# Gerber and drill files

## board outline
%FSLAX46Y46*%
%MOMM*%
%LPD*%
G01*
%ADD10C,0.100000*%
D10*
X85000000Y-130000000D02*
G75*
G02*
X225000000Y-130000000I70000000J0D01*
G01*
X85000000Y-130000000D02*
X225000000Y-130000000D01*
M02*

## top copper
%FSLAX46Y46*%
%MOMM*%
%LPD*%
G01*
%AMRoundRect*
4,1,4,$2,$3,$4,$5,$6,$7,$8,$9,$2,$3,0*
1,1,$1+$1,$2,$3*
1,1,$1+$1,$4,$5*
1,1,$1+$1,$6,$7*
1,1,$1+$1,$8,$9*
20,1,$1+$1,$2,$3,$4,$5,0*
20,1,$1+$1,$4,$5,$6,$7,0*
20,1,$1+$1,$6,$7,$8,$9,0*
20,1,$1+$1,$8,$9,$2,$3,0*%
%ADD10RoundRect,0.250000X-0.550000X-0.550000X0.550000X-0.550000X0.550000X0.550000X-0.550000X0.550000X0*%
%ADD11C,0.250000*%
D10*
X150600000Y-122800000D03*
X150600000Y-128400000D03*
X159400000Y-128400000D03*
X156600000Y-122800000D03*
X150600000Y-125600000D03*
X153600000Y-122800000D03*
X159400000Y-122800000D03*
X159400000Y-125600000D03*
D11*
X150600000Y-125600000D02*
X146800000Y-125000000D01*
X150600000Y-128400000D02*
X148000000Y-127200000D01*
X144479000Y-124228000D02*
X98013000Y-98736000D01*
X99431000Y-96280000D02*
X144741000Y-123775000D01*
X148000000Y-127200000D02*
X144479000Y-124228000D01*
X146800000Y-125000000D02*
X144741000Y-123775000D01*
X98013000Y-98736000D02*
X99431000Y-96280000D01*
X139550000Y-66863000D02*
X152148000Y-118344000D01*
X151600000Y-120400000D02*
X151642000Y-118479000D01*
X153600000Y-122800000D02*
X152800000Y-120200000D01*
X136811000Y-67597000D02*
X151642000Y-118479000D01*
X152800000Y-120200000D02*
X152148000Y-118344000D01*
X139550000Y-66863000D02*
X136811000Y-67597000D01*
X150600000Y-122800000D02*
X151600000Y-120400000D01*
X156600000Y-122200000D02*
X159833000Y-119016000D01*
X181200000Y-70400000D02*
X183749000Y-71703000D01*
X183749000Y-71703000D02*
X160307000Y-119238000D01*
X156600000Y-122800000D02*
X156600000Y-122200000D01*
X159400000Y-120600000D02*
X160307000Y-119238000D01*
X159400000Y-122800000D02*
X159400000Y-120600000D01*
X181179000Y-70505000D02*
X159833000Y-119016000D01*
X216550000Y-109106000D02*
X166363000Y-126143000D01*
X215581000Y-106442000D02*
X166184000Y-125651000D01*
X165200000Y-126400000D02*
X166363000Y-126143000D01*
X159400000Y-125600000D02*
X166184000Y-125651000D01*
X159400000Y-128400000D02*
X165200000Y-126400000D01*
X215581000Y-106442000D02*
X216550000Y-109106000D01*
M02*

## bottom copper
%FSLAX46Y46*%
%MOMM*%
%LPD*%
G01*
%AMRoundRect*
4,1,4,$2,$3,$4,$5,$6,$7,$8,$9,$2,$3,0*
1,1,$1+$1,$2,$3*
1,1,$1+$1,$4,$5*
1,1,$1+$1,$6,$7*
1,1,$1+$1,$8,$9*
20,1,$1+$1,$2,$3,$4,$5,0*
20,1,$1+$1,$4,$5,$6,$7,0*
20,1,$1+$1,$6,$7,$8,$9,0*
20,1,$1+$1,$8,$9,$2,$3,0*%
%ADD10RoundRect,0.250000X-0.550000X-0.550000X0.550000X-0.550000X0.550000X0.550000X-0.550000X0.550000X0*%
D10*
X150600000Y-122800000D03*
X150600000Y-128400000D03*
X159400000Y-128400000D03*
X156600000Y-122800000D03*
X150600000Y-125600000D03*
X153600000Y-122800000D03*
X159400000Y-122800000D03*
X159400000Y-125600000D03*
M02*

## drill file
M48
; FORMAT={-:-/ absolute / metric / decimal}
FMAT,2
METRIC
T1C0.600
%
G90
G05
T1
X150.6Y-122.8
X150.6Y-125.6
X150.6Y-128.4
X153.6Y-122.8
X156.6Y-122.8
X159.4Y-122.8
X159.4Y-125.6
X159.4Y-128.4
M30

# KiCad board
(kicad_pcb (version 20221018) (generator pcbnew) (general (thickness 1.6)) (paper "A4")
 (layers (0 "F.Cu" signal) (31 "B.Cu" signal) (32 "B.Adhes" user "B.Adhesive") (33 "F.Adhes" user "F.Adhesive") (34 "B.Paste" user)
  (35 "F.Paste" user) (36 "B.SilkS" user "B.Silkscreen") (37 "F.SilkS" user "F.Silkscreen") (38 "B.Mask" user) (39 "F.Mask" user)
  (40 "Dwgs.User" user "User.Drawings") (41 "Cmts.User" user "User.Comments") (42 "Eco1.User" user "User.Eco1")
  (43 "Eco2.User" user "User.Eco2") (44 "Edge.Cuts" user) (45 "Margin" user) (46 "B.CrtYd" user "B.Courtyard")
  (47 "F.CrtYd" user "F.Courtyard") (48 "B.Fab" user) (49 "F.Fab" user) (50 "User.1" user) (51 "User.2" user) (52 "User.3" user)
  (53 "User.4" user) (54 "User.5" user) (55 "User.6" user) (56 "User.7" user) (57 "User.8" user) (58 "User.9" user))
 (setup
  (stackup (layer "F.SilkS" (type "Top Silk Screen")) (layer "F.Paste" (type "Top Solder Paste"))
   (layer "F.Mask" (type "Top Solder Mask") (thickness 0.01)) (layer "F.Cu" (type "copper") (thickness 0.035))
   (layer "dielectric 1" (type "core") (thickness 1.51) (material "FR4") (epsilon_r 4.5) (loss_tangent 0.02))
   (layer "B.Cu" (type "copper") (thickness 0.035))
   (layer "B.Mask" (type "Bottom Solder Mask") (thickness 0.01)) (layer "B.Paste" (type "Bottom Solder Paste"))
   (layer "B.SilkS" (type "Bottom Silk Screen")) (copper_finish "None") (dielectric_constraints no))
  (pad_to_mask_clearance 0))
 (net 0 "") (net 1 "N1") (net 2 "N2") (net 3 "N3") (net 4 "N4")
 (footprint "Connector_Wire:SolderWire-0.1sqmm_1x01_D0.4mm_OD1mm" (layer "F.Cu") (at 150.6 122.8)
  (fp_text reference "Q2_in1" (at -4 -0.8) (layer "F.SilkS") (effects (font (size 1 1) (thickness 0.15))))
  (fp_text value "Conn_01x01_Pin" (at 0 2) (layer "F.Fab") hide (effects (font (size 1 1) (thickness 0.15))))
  (pad "1" thru_hole roundrect (at 0 0) (size 1.6 1.6) (drill 0.6) (layers "*.Cu" "*.Mask") (roundrect_rratio 0.15625) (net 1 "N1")))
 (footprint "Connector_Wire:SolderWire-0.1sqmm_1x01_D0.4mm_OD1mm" (layer "F.Cu") (at 150.6 128.4)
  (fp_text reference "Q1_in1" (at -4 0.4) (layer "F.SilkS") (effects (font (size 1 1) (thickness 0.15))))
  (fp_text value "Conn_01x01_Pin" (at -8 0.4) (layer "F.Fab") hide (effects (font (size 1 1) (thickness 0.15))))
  (pad "1" thru_hole roundrect (at 0 0) (size 1.6 1.6) (drill 0.6) (layers "*.Cu" "*.Mask") (roundrect_rratio 0.15625) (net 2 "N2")))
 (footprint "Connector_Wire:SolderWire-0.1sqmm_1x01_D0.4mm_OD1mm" (layer "F.Cu") (at 159.4 128.4)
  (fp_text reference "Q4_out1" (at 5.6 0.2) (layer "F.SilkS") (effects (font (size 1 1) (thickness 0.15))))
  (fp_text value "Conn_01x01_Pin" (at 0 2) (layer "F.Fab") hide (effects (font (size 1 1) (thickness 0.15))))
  (pad "1" thru_hole roundrect (at 0 0) (size 1.6 1.6) (drill 0.6) (layers "*.Cu" "*.Mask") (roundrect_rratio 0.15625) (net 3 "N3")))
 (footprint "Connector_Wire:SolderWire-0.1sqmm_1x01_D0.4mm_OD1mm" (layer "F.Cu") (at 156.6 122.8)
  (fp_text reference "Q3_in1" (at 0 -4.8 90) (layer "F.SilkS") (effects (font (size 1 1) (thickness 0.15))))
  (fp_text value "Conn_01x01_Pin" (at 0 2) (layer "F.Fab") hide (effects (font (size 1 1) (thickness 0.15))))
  (pad "1" thru_hole roundrect (at 0 0) (size 1.6 1.6) (drill 0.6) (layers "*.Cu" "*.Mask") (roundrect_rratio 0.15625) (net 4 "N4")))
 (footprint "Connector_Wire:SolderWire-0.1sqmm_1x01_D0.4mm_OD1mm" (layer "F.Cu") (at 150.6 125.6)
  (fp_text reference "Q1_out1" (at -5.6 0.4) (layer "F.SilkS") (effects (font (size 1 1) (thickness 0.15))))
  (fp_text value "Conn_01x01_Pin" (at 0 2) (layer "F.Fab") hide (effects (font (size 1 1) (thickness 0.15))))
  (pad "1" thru_hole roundrect (at 0 0) (size 1.6 1.6) (drill 0.6) (layers "*.Cu" "*.Mask") (roundrect_rratio 0.15625) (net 2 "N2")))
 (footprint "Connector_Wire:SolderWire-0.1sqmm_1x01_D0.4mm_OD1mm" (layer "F.Cu") (at 153.6 122.8)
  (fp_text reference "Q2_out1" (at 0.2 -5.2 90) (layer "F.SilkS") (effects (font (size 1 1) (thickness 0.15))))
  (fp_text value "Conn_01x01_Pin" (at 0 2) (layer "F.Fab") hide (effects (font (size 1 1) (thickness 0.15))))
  (pad "1" thru_hole roundrect (at 0 0) (size 1.6 1.6) (drill 0.6) (layers "*.Cu" "*.Mask") (roundrect_rratio 0.15625) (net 1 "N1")))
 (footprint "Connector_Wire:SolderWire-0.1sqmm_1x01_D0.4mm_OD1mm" (layer "F.Cu") (at 159.4 122.8)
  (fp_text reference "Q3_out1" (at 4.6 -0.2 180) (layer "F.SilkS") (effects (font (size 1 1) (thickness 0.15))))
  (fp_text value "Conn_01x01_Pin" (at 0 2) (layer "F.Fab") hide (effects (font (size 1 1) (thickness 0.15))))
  (pad "1" thru_hole roundrect (at 0 0) (size 1.6 1.6) (drill 0.6) (layers "*.Cu" "*.Mask") (roundrect_rratio 0.15625) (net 4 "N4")))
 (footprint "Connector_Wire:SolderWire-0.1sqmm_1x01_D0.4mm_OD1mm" (layer "F.Cu") (at 159.4 125.6)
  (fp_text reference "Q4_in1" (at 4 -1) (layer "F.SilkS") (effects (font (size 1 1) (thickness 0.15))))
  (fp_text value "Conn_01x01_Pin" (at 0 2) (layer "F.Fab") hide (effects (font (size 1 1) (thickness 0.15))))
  (pad "1" thru_hole roundrect (at 0 0) (size 1.6 1.6) (drill 0.6) (layers "*.Cu" "*.Mask") (roundrect_rratio 0.15625) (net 3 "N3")))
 (gr_arc (start 85 130) (mid 155 60) (end 225 130) (stroke (width 0.1) (type default)) (layer "Edge.Cuts"))
 (gr_line (start 85 130) (end 225 130) (stroke (width 0.1) (type default)) (layer "Edge.Cuts"))
 (segment (start 150.6 125.6) (end 146.8 125) (width 0.25) (layer "F.Cu") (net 2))
 (segment (start 150.6 128.4) (end 148 127.2) (width 0.25) (layer "F.Cu") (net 2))
 (segment (start 144.479 124.228) (end 98.013 98.736) (width 0.25) (layer "F.Cu") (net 2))
 (segment (start 99.431 96.28) (end 144.741 123.775) (width 0.25) (layer "F.Cu") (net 2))
 (segment (start 148 127.2) (end 144.479 124.228) (width 0.25) (layer "F.Cu") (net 2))
 (segment (start 146.8 125) (end 144.741 123.775) (width 0.25) (layer "F.Cu") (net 2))
 (segment (start 98.013 98.736) (end 99.431 96.28) (width 0.25) (layer "F.Cu") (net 2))
 (segment (start 139.55 66.863) (end 152.148 118.344) (width 0.25) (layer "F.Cu") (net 1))
 (segment (start 151.6 120.4) (end 151.642 118.479) (width 0.25) (layer "F.Cu") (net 1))
 (segment (start 153.6 122.8) (end 152.8 120.2) (width 0.25) (layer "F.Cu") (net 1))
 (segment (start 136.811 67.597) (end 151.642 118.479) (width 0.25) (layer "F.Cu") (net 1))
 (segment (start 152.8 120.2) (end 152.148 118.344) (width 0.25) (layer "F.Cu") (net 1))
 (segment (start 139.55 66.863) (end 136.811 67.597) (width 0.25) (layer "F.Cu") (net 1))
 (segment (start 150.6 122.8) (end 151.6 120.4) (width 0.25) (layer "F.Cu") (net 1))
 (segment (start 156.6 122.2) (end 159.833 119.016) (width 0.25) (layer "F.Cu") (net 4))
 (segment (start 181.2 70.4) (end 183.749 71.703) (width 0.25) (layer "F.Cu") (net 4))
 (segment (start 183.749 71.703) (end 160.307 119.238) (width 0.25) (layer "F.Cu") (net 4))
 (segment (start 156.6 122.8) (end 156.6 122.2) (width 0.25) (layer "F.Cu") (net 4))
 (segment (start 159.4 120.6) (end 160.307 119.238) (width 0.25) (layer "F.Cu") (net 4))
 (segment (start 159.4 122.8) (end 159.4 120.6) (width 0.25) (layer "F.Cu") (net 4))
 (segment (start 181.179 70.505) (end 159.833 119.016) (width 0.25) (layer "F.Cu") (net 4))
 (segment (start 216.55 109.106) (end 166.363 126.143) (width 0.25) (layer "F.Cu") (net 3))
 (segment (start 215.581 106.442) (end 166.184 125.651) (width 0.25) (layer "F.Cu") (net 3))
 (segment (start 165.2 126.4) (end 166.363 126.143) (width 0.25) (layer "F.Cu") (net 3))
 (segment (start 159.4 125.6) (end 166.184 125.651) (width 0.25) (layer "F.Cu") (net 3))
 (segment (start 159.4 128.4) (end 165.2 126.4) (width 0.25) (layer "F.Cu") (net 3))
 (segment (start 215.581 106.442) (end 216.55 109.106) (width 0.25) (layer "F.Cu") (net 3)))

